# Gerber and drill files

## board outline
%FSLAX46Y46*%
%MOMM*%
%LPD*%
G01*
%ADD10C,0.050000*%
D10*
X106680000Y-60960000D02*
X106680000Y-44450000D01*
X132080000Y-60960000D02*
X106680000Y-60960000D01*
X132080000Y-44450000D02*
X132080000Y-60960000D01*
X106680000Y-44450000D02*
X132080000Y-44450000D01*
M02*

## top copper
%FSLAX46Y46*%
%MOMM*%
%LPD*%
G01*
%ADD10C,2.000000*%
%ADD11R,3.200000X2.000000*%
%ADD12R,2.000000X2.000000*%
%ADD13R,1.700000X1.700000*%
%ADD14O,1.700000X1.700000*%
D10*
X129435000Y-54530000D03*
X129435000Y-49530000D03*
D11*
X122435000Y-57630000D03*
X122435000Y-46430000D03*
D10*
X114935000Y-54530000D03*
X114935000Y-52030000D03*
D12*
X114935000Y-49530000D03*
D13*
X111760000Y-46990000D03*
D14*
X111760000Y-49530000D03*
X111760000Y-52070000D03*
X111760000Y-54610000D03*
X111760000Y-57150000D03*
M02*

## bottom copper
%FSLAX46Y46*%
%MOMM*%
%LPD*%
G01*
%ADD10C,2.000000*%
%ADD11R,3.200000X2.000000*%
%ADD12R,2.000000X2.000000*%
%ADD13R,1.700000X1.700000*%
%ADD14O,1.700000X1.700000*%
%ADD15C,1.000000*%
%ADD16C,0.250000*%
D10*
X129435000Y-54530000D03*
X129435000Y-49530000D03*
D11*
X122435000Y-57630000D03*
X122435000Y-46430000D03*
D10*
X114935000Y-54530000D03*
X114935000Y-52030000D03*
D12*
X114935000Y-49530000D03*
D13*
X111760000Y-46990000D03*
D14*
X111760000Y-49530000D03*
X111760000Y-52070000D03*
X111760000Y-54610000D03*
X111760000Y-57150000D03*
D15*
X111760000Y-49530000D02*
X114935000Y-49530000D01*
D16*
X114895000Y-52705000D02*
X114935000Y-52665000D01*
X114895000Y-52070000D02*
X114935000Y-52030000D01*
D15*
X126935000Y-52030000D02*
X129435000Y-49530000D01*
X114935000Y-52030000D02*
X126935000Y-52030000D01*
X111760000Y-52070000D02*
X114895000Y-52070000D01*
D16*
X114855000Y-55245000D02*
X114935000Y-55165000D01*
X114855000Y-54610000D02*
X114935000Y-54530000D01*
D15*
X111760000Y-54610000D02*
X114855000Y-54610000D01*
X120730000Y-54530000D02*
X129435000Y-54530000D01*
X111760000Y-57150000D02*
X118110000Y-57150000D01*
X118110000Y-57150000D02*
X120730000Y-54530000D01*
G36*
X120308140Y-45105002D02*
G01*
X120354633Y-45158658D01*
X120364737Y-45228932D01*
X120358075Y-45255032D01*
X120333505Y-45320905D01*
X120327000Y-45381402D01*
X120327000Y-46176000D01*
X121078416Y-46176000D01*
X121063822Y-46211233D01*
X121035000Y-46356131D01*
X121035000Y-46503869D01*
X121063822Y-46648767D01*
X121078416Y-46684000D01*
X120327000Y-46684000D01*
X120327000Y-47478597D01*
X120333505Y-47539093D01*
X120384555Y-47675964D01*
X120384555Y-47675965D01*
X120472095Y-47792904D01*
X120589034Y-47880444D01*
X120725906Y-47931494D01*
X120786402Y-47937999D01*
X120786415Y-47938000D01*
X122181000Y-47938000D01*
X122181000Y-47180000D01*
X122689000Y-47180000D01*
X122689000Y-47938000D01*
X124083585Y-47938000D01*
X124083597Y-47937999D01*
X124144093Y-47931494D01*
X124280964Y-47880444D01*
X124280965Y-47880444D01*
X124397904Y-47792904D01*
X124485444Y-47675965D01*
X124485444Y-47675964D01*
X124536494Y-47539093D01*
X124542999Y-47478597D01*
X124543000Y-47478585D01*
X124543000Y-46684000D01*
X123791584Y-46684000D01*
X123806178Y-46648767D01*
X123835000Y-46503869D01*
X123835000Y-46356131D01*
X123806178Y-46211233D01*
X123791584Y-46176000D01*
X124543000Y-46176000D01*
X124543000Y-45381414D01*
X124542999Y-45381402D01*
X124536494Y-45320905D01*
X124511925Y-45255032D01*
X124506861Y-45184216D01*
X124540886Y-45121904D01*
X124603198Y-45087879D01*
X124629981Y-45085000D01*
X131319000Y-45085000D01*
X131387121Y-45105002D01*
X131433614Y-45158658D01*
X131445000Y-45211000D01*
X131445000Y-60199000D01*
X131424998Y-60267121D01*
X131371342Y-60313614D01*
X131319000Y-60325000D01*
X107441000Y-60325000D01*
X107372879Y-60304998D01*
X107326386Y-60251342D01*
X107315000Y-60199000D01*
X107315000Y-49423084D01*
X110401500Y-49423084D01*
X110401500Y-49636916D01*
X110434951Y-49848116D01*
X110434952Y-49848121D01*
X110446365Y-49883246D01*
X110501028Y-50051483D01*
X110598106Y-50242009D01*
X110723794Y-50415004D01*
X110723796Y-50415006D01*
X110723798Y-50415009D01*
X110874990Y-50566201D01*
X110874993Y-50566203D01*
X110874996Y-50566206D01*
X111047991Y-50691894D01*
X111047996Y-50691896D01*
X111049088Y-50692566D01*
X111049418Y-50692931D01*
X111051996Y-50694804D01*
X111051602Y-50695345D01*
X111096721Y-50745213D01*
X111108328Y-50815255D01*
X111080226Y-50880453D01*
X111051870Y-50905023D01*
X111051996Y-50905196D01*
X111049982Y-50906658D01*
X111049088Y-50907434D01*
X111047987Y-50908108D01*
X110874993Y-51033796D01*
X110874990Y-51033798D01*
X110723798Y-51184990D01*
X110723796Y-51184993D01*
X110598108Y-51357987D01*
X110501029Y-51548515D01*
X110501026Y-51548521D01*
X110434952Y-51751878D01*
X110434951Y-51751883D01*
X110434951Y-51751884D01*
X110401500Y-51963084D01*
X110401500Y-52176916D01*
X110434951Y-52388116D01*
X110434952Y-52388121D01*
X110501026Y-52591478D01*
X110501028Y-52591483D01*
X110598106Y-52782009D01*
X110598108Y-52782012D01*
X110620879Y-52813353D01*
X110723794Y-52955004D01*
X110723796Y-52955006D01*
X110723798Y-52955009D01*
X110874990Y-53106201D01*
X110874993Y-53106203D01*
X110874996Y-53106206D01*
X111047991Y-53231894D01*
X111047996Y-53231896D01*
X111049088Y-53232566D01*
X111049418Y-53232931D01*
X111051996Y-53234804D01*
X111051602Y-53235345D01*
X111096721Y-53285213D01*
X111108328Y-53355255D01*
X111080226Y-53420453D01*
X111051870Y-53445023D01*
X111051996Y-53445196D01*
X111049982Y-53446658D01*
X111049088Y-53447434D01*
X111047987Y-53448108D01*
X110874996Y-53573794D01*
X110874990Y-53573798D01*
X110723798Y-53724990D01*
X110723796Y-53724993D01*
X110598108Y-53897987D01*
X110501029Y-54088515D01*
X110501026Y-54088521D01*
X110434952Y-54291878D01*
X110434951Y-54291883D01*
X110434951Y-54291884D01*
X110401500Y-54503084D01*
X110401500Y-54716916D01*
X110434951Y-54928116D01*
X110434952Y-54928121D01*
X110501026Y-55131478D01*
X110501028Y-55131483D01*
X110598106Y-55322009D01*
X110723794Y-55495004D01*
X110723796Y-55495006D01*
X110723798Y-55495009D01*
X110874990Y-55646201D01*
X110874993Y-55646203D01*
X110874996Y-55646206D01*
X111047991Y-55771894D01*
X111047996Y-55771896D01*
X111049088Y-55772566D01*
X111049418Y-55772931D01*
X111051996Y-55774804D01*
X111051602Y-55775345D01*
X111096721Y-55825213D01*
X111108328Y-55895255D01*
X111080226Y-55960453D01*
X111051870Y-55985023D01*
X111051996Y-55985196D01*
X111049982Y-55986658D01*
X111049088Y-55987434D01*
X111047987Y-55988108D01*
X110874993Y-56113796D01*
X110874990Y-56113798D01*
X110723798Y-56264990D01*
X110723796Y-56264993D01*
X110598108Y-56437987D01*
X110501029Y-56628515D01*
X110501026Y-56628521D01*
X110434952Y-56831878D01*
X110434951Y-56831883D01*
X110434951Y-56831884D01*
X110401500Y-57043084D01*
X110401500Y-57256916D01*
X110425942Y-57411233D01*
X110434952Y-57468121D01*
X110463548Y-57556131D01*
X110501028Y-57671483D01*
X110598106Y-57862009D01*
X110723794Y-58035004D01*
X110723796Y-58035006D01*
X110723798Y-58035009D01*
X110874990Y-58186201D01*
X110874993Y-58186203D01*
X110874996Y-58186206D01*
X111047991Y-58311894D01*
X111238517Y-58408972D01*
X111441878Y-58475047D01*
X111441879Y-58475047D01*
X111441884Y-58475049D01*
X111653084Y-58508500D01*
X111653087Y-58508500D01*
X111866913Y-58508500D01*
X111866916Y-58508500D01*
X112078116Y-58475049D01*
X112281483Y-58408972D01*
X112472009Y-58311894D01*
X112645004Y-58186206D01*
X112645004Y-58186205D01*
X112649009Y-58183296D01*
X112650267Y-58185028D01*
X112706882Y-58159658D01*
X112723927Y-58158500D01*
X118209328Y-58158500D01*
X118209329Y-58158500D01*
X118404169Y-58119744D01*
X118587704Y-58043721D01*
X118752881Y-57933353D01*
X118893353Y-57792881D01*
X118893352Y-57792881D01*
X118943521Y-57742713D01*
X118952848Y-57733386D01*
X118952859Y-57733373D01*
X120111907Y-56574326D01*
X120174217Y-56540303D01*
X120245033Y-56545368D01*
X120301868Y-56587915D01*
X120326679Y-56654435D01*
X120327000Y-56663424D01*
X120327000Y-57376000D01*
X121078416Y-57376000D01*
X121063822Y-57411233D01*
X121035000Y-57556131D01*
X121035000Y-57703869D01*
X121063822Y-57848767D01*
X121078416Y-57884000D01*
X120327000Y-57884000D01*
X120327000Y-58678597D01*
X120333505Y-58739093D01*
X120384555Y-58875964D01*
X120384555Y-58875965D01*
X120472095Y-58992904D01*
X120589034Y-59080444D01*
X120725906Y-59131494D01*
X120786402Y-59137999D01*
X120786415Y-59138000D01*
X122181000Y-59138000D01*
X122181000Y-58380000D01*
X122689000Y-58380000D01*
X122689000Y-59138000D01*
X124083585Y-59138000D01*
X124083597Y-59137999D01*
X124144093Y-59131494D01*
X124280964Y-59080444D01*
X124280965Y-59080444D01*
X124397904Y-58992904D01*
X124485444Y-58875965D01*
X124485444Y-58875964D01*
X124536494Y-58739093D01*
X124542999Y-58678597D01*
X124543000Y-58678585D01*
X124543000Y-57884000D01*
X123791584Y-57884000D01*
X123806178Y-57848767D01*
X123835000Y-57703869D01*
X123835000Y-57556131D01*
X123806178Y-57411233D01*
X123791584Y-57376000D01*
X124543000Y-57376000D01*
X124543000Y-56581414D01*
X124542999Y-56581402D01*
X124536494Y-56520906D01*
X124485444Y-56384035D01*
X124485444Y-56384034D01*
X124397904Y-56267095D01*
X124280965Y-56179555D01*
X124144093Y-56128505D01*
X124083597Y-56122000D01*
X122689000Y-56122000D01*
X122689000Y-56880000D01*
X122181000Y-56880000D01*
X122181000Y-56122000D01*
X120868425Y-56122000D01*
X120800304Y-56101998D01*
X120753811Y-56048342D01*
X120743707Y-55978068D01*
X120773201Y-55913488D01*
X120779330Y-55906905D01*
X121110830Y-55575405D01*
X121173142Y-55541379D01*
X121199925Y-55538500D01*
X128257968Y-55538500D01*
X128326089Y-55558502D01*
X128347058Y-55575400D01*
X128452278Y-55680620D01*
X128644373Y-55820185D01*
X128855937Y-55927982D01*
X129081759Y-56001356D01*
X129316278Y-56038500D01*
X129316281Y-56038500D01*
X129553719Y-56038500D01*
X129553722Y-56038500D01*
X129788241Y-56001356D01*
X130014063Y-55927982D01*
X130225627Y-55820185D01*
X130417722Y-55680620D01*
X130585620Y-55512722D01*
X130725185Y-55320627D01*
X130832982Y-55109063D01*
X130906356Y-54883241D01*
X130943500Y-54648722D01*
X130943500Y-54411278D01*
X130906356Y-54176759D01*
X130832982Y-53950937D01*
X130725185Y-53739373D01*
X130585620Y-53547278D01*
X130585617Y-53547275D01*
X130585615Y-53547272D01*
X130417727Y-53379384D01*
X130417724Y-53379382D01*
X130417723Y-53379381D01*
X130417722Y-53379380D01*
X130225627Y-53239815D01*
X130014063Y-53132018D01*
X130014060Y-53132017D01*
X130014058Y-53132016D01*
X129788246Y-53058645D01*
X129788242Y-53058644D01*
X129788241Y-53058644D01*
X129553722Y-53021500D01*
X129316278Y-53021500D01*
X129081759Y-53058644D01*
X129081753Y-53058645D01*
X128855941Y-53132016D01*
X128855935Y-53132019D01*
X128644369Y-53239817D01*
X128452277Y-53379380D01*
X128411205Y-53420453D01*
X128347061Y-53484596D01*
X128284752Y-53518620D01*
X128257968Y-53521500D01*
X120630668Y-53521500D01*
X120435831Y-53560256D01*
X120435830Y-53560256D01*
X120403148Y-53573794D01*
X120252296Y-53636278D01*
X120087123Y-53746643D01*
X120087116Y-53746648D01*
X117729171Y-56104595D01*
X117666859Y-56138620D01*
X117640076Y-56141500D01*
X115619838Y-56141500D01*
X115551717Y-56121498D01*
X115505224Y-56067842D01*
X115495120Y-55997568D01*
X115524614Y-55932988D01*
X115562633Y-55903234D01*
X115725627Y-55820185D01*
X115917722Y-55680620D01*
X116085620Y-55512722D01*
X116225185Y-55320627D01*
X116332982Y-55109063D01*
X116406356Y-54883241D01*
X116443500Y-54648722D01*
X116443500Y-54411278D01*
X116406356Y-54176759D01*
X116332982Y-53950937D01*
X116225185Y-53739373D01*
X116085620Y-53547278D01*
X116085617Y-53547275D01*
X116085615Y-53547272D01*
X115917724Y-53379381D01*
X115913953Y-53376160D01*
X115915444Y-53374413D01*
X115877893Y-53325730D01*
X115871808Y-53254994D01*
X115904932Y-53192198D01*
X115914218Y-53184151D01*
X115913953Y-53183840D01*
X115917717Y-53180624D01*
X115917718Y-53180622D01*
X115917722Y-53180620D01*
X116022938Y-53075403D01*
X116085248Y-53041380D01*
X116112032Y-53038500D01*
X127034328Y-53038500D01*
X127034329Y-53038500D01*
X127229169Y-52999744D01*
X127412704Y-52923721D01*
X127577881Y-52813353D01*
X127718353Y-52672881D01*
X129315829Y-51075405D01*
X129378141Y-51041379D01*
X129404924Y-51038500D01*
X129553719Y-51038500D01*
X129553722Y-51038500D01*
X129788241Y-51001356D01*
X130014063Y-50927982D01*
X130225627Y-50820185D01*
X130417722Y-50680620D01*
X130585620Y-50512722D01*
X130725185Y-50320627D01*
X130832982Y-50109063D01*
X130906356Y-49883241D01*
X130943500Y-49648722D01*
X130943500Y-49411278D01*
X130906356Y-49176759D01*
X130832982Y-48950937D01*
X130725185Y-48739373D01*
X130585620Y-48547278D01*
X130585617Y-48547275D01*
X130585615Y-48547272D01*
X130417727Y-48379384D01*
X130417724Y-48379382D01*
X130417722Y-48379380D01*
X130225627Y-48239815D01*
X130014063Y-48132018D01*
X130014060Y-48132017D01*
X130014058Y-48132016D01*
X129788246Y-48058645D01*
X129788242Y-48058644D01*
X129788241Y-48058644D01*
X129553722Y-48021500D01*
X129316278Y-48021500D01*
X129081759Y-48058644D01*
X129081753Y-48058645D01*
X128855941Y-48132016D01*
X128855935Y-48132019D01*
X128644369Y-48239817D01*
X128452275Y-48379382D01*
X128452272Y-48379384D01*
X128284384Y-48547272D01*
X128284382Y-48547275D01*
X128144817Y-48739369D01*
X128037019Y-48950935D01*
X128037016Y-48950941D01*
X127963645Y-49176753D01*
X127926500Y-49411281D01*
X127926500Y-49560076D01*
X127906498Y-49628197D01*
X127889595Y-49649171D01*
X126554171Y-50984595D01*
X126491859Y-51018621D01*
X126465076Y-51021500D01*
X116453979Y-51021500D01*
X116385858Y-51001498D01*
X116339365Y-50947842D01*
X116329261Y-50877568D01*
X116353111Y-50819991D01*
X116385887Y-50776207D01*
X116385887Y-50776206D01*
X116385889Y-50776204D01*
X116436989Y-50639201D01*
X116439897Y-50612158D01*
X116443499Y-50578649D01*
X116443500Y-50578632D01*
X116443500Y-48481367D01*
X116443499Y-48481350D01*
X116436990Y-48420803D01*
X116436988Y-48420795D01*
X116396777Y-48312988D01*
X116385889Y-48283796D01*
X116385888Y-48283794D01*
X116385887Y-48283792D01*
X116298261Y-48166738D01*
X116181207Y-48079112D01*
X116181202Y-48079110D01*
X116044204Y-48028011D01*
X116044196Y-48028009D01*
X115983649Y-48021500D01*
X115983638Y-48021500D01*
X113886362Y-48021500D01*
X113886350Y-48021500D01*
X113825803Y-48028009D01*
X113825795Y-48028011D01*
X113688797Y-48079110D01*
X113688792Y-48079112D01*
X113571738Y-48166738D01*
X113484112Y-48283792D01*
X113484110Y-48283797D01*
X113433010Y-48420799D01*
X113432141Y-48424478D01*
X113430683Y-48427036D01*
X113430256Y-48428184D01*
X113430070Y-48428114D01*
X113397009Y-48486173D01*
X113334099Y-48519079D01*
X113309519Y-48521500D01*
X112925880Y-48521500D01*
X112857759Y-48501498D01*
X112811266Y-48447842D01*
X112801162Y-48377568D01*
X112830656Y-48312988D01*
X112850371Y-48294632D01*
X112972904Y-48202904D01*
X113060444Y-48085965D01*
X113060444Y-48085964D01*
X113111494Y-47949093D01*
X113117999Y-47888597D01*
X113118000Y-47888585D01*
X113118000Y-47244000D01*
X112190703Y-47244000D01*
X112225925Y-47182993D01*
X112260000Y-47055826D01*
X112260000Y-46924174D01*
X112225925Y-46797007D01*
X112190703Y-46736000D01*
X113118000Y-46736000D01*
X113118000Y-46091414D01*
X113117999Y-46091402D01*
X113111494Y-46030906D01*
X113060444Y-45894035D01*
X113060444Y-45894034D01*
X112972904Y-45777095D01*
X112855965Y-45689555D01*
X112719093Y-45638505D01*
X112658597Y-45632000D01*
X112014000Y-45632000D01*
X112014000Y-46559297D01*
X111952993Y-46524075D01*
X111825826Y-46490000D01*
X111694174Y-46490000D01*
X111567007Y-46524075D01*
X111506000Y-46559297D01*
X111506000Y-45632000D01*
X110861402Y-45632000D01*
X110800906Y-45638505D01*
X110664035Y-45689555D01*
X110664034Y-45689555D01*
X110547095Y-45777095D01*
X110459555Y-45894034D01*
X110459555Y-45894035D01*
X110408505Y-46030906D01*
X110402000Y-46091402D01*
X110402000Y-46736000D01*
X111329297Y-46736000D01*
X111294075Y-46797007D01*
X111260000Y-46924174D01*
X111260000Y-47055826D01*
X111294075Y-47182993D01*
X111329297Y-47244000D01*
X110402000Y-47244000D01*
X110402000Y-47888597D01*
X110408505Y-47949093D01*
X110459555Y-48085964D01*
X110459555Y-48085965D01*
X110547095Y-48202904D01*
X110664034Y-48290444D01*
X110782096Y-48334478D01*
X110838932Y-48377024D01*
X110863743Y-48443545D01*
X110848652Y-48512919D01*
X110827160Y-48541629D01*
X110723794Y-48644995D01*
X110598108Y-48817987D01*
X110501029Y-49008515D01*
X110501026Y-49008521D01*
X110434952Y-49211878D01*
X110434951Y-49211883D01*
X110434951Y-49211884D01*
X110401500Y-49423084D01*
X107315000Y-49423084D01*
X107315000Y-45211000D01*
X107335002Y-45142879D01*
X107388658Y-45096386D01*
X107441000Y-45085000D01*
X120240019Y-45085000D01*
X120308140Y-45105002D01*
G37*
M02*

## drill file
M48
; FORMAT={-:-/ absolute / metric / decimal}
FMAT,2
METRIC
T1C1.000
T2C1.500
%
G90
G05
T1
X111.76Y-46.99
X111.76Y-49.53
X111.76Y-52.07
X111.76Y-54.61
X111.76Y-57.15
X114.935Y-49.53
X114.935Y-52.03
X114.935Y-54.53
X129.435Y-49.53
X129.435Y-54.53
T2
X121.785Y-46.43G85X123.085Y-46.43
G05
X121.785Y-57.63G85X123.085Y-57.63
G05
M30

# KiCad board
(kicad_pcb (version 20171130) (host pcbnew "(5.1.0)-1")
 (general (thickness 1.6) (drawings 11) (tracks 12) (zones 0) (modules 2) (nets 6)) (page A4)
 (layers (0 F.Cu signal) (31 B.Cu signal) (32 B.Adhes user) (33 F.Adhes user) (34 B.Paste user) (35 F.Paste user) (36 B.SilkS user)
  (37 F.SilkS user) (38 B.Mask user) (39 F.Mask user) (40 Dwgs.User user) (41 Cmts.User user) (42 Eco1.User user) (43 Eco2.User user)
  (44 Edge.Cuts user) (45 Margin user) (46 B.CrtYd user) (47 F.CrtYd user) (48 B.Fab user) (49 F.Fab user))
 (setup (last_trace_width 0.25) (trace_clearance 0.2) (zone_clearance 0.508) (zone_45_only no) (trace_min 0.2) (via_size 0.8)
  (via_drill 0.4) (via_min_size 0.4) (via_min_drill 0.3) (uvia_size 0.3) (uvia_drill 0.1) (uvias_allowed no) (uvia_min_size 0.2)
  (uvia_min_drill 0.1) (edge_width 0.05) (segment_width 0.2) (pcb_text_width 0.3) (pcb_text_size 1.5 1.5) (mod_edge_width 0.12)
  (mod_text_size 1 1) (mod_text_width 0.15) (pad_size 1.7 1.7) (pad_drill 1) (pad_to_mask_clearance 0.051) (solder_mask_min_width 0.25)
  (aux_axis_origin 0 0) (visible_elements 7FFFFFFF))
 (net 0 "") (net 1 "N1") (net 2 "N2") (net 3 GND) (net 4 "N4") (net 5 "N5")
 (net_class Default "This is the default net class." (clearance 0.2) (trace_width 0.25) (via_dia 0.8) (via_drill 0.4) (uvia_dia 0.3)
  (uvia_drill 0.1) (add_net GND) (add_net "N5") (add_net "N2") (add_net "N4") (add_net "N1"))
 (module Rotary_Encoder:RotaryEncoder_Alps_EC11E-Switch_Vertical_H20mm (layer F.Cu) (at 114.935 49.53)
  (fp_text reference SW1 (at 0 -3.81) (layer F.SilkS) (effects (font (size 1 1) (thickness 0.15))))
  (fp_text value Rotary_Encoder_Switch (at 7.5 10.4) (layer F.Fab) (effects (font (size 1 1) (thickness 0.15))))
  (pad S1 thru_hole circle (at 14.5 5) (size 2 2) (drill 1) (layers *.Cu *.Mask) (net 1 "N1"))
  (pad S2 thru_hole circle (at 14.5 0) (size 2 2) (drill 1) (layers *.Cu *.Mask) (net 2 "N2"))
  (pad MP thru_hole rect (at 7.5 8.1) (size 3.2 2) (drill oval 2.8 1.5) (layers *.Cu *.Mask) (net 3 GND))
  (pad MP thru_hole rect (at 7.5 -3.1) (size 3.2 2) (drill oval 2.8 1.5) (layers *.Cu *.Mask) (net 3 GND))
  (pad B thru_hole circle (at 0 5) (size 2 2) (drill 1) (layers *.Cu *.Mask) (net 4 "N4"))
  (pad C thru_hole circle (at 0 2.5) (size 2 2) (drill 1) (layers *.Cu *.Mask) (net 2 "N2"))
  (pad A thru_hole rect (at 0 0) (size 2 2) (drill 1) (layers *.Cu *.Mask) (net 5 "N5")))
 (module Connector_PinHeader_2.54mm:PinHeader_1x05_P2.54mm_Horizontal (layer B.Cu) (at 111.76 46.99 180)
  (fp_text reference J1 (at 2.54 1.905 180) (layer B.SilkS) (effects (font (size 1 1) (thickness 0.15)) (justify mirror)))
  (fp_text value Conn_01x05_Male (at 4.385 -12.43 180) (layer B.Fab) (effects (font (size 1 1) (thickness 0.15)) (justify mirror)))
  (pad 1 thru_hole rect (at 0 0 180) (size 1.7 1.7) (drill 1) (layers *.Cu *.Mask) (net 3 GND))
  (pad 2 thru_hole oval (at 0 -2.54 180) (size 1.7 1.7) (drill 1) (layers *.Cu *.Mask) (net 5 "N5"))
  (pad 3 thru_hole oval (at 0 -5.08 180) (size 1.7 1.7) (drill 1) (layers *.Cu *.Mask) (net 2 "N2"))
  (pad 4 thru_hole oval (at 0 -7.62 180) (size 1.7 1.7) (drill 1) (layers *.Cu *.Mask) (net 4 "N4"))
  (pad 5 thru_hole oval (at 0 -10.16 180) (size 1.7 1.7) (drill 1) (layers *.Cu *.Mask) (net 1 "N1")))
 (gr_line (start 106.68 60.96) (end 106.68 44.45) (layer Edge.Cuts) (width 0.05))
 (gr_line (start 132.08 60.96) (end 106.68 60.96) (layer Edge.Cuts) (width 0.05))
 (gr_line (start 132.08 44.45) (end 132.08 60.96) (layer Edge.Cuts) (width 0.05))
 (gr_line (start 106.68 44.45) (end 132.08 44.45) (layer Edge.Cuts) (width 0.05))
 (segment (start 111.76 49.53) (end 114.935 49.53) (width 1) (layer B.Cu) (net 5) (status 30))
 (segment (start 114.895 52.705) (end 114.935 52.665) (width 0.25) (layer B.Cu) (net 2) (status 30))
 (segment (start 114.895 52.07) (end 114.935 52.03) (width 0.25) (layer B.Cu) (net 2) (status 30))
 (segment (start 126.935 52.03) (end 129.435 49.53) (width 1) (layer B.Cu) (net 2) (status 20))
 (segment (start 114.935 52.03) (end 126.935 52.03) (width 1) (layer B.Cu) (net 2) (status 10))
 (segment (start 111.76 52.07) (end 114.895 52.07) (width 1) (layer B.Cu) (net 2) (status 30))
 (segment (start 114.855 55.245) (end 114.935 55.165) (width 0.25) (layer B.Cu) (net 4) (status 30))
 (segment (start 114.855 54.61) (end 114.935 54.53) (width 0.25) (layer B.Cu) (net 4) (status 30))
 (segment (start 111.76 54.61) (end 114.855 54.61) (width 1) (layer B.Cu) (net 4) (status 30))
 (segment (start 120.73 54.53) (end 129.435 54.53) (width 1) (layer B.Cu) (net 1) (status 20))
 (segment (start 111.76 57.15) (end 118.11 57.15) (width 1) (layer B.Cu) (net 1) (status 10))
 (segment (start 118.11 57.15) (end 120.73 54.53) (width 1) (layer B.Cu) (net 1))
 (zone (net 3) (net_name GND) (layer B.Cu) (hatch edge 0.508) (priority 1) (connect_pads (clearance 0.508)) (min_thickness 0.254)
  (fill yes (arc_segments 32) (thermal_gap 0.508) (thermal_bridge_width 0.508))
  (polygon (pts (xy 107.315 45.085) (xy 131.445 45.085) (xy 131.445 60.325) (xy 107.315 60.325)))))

